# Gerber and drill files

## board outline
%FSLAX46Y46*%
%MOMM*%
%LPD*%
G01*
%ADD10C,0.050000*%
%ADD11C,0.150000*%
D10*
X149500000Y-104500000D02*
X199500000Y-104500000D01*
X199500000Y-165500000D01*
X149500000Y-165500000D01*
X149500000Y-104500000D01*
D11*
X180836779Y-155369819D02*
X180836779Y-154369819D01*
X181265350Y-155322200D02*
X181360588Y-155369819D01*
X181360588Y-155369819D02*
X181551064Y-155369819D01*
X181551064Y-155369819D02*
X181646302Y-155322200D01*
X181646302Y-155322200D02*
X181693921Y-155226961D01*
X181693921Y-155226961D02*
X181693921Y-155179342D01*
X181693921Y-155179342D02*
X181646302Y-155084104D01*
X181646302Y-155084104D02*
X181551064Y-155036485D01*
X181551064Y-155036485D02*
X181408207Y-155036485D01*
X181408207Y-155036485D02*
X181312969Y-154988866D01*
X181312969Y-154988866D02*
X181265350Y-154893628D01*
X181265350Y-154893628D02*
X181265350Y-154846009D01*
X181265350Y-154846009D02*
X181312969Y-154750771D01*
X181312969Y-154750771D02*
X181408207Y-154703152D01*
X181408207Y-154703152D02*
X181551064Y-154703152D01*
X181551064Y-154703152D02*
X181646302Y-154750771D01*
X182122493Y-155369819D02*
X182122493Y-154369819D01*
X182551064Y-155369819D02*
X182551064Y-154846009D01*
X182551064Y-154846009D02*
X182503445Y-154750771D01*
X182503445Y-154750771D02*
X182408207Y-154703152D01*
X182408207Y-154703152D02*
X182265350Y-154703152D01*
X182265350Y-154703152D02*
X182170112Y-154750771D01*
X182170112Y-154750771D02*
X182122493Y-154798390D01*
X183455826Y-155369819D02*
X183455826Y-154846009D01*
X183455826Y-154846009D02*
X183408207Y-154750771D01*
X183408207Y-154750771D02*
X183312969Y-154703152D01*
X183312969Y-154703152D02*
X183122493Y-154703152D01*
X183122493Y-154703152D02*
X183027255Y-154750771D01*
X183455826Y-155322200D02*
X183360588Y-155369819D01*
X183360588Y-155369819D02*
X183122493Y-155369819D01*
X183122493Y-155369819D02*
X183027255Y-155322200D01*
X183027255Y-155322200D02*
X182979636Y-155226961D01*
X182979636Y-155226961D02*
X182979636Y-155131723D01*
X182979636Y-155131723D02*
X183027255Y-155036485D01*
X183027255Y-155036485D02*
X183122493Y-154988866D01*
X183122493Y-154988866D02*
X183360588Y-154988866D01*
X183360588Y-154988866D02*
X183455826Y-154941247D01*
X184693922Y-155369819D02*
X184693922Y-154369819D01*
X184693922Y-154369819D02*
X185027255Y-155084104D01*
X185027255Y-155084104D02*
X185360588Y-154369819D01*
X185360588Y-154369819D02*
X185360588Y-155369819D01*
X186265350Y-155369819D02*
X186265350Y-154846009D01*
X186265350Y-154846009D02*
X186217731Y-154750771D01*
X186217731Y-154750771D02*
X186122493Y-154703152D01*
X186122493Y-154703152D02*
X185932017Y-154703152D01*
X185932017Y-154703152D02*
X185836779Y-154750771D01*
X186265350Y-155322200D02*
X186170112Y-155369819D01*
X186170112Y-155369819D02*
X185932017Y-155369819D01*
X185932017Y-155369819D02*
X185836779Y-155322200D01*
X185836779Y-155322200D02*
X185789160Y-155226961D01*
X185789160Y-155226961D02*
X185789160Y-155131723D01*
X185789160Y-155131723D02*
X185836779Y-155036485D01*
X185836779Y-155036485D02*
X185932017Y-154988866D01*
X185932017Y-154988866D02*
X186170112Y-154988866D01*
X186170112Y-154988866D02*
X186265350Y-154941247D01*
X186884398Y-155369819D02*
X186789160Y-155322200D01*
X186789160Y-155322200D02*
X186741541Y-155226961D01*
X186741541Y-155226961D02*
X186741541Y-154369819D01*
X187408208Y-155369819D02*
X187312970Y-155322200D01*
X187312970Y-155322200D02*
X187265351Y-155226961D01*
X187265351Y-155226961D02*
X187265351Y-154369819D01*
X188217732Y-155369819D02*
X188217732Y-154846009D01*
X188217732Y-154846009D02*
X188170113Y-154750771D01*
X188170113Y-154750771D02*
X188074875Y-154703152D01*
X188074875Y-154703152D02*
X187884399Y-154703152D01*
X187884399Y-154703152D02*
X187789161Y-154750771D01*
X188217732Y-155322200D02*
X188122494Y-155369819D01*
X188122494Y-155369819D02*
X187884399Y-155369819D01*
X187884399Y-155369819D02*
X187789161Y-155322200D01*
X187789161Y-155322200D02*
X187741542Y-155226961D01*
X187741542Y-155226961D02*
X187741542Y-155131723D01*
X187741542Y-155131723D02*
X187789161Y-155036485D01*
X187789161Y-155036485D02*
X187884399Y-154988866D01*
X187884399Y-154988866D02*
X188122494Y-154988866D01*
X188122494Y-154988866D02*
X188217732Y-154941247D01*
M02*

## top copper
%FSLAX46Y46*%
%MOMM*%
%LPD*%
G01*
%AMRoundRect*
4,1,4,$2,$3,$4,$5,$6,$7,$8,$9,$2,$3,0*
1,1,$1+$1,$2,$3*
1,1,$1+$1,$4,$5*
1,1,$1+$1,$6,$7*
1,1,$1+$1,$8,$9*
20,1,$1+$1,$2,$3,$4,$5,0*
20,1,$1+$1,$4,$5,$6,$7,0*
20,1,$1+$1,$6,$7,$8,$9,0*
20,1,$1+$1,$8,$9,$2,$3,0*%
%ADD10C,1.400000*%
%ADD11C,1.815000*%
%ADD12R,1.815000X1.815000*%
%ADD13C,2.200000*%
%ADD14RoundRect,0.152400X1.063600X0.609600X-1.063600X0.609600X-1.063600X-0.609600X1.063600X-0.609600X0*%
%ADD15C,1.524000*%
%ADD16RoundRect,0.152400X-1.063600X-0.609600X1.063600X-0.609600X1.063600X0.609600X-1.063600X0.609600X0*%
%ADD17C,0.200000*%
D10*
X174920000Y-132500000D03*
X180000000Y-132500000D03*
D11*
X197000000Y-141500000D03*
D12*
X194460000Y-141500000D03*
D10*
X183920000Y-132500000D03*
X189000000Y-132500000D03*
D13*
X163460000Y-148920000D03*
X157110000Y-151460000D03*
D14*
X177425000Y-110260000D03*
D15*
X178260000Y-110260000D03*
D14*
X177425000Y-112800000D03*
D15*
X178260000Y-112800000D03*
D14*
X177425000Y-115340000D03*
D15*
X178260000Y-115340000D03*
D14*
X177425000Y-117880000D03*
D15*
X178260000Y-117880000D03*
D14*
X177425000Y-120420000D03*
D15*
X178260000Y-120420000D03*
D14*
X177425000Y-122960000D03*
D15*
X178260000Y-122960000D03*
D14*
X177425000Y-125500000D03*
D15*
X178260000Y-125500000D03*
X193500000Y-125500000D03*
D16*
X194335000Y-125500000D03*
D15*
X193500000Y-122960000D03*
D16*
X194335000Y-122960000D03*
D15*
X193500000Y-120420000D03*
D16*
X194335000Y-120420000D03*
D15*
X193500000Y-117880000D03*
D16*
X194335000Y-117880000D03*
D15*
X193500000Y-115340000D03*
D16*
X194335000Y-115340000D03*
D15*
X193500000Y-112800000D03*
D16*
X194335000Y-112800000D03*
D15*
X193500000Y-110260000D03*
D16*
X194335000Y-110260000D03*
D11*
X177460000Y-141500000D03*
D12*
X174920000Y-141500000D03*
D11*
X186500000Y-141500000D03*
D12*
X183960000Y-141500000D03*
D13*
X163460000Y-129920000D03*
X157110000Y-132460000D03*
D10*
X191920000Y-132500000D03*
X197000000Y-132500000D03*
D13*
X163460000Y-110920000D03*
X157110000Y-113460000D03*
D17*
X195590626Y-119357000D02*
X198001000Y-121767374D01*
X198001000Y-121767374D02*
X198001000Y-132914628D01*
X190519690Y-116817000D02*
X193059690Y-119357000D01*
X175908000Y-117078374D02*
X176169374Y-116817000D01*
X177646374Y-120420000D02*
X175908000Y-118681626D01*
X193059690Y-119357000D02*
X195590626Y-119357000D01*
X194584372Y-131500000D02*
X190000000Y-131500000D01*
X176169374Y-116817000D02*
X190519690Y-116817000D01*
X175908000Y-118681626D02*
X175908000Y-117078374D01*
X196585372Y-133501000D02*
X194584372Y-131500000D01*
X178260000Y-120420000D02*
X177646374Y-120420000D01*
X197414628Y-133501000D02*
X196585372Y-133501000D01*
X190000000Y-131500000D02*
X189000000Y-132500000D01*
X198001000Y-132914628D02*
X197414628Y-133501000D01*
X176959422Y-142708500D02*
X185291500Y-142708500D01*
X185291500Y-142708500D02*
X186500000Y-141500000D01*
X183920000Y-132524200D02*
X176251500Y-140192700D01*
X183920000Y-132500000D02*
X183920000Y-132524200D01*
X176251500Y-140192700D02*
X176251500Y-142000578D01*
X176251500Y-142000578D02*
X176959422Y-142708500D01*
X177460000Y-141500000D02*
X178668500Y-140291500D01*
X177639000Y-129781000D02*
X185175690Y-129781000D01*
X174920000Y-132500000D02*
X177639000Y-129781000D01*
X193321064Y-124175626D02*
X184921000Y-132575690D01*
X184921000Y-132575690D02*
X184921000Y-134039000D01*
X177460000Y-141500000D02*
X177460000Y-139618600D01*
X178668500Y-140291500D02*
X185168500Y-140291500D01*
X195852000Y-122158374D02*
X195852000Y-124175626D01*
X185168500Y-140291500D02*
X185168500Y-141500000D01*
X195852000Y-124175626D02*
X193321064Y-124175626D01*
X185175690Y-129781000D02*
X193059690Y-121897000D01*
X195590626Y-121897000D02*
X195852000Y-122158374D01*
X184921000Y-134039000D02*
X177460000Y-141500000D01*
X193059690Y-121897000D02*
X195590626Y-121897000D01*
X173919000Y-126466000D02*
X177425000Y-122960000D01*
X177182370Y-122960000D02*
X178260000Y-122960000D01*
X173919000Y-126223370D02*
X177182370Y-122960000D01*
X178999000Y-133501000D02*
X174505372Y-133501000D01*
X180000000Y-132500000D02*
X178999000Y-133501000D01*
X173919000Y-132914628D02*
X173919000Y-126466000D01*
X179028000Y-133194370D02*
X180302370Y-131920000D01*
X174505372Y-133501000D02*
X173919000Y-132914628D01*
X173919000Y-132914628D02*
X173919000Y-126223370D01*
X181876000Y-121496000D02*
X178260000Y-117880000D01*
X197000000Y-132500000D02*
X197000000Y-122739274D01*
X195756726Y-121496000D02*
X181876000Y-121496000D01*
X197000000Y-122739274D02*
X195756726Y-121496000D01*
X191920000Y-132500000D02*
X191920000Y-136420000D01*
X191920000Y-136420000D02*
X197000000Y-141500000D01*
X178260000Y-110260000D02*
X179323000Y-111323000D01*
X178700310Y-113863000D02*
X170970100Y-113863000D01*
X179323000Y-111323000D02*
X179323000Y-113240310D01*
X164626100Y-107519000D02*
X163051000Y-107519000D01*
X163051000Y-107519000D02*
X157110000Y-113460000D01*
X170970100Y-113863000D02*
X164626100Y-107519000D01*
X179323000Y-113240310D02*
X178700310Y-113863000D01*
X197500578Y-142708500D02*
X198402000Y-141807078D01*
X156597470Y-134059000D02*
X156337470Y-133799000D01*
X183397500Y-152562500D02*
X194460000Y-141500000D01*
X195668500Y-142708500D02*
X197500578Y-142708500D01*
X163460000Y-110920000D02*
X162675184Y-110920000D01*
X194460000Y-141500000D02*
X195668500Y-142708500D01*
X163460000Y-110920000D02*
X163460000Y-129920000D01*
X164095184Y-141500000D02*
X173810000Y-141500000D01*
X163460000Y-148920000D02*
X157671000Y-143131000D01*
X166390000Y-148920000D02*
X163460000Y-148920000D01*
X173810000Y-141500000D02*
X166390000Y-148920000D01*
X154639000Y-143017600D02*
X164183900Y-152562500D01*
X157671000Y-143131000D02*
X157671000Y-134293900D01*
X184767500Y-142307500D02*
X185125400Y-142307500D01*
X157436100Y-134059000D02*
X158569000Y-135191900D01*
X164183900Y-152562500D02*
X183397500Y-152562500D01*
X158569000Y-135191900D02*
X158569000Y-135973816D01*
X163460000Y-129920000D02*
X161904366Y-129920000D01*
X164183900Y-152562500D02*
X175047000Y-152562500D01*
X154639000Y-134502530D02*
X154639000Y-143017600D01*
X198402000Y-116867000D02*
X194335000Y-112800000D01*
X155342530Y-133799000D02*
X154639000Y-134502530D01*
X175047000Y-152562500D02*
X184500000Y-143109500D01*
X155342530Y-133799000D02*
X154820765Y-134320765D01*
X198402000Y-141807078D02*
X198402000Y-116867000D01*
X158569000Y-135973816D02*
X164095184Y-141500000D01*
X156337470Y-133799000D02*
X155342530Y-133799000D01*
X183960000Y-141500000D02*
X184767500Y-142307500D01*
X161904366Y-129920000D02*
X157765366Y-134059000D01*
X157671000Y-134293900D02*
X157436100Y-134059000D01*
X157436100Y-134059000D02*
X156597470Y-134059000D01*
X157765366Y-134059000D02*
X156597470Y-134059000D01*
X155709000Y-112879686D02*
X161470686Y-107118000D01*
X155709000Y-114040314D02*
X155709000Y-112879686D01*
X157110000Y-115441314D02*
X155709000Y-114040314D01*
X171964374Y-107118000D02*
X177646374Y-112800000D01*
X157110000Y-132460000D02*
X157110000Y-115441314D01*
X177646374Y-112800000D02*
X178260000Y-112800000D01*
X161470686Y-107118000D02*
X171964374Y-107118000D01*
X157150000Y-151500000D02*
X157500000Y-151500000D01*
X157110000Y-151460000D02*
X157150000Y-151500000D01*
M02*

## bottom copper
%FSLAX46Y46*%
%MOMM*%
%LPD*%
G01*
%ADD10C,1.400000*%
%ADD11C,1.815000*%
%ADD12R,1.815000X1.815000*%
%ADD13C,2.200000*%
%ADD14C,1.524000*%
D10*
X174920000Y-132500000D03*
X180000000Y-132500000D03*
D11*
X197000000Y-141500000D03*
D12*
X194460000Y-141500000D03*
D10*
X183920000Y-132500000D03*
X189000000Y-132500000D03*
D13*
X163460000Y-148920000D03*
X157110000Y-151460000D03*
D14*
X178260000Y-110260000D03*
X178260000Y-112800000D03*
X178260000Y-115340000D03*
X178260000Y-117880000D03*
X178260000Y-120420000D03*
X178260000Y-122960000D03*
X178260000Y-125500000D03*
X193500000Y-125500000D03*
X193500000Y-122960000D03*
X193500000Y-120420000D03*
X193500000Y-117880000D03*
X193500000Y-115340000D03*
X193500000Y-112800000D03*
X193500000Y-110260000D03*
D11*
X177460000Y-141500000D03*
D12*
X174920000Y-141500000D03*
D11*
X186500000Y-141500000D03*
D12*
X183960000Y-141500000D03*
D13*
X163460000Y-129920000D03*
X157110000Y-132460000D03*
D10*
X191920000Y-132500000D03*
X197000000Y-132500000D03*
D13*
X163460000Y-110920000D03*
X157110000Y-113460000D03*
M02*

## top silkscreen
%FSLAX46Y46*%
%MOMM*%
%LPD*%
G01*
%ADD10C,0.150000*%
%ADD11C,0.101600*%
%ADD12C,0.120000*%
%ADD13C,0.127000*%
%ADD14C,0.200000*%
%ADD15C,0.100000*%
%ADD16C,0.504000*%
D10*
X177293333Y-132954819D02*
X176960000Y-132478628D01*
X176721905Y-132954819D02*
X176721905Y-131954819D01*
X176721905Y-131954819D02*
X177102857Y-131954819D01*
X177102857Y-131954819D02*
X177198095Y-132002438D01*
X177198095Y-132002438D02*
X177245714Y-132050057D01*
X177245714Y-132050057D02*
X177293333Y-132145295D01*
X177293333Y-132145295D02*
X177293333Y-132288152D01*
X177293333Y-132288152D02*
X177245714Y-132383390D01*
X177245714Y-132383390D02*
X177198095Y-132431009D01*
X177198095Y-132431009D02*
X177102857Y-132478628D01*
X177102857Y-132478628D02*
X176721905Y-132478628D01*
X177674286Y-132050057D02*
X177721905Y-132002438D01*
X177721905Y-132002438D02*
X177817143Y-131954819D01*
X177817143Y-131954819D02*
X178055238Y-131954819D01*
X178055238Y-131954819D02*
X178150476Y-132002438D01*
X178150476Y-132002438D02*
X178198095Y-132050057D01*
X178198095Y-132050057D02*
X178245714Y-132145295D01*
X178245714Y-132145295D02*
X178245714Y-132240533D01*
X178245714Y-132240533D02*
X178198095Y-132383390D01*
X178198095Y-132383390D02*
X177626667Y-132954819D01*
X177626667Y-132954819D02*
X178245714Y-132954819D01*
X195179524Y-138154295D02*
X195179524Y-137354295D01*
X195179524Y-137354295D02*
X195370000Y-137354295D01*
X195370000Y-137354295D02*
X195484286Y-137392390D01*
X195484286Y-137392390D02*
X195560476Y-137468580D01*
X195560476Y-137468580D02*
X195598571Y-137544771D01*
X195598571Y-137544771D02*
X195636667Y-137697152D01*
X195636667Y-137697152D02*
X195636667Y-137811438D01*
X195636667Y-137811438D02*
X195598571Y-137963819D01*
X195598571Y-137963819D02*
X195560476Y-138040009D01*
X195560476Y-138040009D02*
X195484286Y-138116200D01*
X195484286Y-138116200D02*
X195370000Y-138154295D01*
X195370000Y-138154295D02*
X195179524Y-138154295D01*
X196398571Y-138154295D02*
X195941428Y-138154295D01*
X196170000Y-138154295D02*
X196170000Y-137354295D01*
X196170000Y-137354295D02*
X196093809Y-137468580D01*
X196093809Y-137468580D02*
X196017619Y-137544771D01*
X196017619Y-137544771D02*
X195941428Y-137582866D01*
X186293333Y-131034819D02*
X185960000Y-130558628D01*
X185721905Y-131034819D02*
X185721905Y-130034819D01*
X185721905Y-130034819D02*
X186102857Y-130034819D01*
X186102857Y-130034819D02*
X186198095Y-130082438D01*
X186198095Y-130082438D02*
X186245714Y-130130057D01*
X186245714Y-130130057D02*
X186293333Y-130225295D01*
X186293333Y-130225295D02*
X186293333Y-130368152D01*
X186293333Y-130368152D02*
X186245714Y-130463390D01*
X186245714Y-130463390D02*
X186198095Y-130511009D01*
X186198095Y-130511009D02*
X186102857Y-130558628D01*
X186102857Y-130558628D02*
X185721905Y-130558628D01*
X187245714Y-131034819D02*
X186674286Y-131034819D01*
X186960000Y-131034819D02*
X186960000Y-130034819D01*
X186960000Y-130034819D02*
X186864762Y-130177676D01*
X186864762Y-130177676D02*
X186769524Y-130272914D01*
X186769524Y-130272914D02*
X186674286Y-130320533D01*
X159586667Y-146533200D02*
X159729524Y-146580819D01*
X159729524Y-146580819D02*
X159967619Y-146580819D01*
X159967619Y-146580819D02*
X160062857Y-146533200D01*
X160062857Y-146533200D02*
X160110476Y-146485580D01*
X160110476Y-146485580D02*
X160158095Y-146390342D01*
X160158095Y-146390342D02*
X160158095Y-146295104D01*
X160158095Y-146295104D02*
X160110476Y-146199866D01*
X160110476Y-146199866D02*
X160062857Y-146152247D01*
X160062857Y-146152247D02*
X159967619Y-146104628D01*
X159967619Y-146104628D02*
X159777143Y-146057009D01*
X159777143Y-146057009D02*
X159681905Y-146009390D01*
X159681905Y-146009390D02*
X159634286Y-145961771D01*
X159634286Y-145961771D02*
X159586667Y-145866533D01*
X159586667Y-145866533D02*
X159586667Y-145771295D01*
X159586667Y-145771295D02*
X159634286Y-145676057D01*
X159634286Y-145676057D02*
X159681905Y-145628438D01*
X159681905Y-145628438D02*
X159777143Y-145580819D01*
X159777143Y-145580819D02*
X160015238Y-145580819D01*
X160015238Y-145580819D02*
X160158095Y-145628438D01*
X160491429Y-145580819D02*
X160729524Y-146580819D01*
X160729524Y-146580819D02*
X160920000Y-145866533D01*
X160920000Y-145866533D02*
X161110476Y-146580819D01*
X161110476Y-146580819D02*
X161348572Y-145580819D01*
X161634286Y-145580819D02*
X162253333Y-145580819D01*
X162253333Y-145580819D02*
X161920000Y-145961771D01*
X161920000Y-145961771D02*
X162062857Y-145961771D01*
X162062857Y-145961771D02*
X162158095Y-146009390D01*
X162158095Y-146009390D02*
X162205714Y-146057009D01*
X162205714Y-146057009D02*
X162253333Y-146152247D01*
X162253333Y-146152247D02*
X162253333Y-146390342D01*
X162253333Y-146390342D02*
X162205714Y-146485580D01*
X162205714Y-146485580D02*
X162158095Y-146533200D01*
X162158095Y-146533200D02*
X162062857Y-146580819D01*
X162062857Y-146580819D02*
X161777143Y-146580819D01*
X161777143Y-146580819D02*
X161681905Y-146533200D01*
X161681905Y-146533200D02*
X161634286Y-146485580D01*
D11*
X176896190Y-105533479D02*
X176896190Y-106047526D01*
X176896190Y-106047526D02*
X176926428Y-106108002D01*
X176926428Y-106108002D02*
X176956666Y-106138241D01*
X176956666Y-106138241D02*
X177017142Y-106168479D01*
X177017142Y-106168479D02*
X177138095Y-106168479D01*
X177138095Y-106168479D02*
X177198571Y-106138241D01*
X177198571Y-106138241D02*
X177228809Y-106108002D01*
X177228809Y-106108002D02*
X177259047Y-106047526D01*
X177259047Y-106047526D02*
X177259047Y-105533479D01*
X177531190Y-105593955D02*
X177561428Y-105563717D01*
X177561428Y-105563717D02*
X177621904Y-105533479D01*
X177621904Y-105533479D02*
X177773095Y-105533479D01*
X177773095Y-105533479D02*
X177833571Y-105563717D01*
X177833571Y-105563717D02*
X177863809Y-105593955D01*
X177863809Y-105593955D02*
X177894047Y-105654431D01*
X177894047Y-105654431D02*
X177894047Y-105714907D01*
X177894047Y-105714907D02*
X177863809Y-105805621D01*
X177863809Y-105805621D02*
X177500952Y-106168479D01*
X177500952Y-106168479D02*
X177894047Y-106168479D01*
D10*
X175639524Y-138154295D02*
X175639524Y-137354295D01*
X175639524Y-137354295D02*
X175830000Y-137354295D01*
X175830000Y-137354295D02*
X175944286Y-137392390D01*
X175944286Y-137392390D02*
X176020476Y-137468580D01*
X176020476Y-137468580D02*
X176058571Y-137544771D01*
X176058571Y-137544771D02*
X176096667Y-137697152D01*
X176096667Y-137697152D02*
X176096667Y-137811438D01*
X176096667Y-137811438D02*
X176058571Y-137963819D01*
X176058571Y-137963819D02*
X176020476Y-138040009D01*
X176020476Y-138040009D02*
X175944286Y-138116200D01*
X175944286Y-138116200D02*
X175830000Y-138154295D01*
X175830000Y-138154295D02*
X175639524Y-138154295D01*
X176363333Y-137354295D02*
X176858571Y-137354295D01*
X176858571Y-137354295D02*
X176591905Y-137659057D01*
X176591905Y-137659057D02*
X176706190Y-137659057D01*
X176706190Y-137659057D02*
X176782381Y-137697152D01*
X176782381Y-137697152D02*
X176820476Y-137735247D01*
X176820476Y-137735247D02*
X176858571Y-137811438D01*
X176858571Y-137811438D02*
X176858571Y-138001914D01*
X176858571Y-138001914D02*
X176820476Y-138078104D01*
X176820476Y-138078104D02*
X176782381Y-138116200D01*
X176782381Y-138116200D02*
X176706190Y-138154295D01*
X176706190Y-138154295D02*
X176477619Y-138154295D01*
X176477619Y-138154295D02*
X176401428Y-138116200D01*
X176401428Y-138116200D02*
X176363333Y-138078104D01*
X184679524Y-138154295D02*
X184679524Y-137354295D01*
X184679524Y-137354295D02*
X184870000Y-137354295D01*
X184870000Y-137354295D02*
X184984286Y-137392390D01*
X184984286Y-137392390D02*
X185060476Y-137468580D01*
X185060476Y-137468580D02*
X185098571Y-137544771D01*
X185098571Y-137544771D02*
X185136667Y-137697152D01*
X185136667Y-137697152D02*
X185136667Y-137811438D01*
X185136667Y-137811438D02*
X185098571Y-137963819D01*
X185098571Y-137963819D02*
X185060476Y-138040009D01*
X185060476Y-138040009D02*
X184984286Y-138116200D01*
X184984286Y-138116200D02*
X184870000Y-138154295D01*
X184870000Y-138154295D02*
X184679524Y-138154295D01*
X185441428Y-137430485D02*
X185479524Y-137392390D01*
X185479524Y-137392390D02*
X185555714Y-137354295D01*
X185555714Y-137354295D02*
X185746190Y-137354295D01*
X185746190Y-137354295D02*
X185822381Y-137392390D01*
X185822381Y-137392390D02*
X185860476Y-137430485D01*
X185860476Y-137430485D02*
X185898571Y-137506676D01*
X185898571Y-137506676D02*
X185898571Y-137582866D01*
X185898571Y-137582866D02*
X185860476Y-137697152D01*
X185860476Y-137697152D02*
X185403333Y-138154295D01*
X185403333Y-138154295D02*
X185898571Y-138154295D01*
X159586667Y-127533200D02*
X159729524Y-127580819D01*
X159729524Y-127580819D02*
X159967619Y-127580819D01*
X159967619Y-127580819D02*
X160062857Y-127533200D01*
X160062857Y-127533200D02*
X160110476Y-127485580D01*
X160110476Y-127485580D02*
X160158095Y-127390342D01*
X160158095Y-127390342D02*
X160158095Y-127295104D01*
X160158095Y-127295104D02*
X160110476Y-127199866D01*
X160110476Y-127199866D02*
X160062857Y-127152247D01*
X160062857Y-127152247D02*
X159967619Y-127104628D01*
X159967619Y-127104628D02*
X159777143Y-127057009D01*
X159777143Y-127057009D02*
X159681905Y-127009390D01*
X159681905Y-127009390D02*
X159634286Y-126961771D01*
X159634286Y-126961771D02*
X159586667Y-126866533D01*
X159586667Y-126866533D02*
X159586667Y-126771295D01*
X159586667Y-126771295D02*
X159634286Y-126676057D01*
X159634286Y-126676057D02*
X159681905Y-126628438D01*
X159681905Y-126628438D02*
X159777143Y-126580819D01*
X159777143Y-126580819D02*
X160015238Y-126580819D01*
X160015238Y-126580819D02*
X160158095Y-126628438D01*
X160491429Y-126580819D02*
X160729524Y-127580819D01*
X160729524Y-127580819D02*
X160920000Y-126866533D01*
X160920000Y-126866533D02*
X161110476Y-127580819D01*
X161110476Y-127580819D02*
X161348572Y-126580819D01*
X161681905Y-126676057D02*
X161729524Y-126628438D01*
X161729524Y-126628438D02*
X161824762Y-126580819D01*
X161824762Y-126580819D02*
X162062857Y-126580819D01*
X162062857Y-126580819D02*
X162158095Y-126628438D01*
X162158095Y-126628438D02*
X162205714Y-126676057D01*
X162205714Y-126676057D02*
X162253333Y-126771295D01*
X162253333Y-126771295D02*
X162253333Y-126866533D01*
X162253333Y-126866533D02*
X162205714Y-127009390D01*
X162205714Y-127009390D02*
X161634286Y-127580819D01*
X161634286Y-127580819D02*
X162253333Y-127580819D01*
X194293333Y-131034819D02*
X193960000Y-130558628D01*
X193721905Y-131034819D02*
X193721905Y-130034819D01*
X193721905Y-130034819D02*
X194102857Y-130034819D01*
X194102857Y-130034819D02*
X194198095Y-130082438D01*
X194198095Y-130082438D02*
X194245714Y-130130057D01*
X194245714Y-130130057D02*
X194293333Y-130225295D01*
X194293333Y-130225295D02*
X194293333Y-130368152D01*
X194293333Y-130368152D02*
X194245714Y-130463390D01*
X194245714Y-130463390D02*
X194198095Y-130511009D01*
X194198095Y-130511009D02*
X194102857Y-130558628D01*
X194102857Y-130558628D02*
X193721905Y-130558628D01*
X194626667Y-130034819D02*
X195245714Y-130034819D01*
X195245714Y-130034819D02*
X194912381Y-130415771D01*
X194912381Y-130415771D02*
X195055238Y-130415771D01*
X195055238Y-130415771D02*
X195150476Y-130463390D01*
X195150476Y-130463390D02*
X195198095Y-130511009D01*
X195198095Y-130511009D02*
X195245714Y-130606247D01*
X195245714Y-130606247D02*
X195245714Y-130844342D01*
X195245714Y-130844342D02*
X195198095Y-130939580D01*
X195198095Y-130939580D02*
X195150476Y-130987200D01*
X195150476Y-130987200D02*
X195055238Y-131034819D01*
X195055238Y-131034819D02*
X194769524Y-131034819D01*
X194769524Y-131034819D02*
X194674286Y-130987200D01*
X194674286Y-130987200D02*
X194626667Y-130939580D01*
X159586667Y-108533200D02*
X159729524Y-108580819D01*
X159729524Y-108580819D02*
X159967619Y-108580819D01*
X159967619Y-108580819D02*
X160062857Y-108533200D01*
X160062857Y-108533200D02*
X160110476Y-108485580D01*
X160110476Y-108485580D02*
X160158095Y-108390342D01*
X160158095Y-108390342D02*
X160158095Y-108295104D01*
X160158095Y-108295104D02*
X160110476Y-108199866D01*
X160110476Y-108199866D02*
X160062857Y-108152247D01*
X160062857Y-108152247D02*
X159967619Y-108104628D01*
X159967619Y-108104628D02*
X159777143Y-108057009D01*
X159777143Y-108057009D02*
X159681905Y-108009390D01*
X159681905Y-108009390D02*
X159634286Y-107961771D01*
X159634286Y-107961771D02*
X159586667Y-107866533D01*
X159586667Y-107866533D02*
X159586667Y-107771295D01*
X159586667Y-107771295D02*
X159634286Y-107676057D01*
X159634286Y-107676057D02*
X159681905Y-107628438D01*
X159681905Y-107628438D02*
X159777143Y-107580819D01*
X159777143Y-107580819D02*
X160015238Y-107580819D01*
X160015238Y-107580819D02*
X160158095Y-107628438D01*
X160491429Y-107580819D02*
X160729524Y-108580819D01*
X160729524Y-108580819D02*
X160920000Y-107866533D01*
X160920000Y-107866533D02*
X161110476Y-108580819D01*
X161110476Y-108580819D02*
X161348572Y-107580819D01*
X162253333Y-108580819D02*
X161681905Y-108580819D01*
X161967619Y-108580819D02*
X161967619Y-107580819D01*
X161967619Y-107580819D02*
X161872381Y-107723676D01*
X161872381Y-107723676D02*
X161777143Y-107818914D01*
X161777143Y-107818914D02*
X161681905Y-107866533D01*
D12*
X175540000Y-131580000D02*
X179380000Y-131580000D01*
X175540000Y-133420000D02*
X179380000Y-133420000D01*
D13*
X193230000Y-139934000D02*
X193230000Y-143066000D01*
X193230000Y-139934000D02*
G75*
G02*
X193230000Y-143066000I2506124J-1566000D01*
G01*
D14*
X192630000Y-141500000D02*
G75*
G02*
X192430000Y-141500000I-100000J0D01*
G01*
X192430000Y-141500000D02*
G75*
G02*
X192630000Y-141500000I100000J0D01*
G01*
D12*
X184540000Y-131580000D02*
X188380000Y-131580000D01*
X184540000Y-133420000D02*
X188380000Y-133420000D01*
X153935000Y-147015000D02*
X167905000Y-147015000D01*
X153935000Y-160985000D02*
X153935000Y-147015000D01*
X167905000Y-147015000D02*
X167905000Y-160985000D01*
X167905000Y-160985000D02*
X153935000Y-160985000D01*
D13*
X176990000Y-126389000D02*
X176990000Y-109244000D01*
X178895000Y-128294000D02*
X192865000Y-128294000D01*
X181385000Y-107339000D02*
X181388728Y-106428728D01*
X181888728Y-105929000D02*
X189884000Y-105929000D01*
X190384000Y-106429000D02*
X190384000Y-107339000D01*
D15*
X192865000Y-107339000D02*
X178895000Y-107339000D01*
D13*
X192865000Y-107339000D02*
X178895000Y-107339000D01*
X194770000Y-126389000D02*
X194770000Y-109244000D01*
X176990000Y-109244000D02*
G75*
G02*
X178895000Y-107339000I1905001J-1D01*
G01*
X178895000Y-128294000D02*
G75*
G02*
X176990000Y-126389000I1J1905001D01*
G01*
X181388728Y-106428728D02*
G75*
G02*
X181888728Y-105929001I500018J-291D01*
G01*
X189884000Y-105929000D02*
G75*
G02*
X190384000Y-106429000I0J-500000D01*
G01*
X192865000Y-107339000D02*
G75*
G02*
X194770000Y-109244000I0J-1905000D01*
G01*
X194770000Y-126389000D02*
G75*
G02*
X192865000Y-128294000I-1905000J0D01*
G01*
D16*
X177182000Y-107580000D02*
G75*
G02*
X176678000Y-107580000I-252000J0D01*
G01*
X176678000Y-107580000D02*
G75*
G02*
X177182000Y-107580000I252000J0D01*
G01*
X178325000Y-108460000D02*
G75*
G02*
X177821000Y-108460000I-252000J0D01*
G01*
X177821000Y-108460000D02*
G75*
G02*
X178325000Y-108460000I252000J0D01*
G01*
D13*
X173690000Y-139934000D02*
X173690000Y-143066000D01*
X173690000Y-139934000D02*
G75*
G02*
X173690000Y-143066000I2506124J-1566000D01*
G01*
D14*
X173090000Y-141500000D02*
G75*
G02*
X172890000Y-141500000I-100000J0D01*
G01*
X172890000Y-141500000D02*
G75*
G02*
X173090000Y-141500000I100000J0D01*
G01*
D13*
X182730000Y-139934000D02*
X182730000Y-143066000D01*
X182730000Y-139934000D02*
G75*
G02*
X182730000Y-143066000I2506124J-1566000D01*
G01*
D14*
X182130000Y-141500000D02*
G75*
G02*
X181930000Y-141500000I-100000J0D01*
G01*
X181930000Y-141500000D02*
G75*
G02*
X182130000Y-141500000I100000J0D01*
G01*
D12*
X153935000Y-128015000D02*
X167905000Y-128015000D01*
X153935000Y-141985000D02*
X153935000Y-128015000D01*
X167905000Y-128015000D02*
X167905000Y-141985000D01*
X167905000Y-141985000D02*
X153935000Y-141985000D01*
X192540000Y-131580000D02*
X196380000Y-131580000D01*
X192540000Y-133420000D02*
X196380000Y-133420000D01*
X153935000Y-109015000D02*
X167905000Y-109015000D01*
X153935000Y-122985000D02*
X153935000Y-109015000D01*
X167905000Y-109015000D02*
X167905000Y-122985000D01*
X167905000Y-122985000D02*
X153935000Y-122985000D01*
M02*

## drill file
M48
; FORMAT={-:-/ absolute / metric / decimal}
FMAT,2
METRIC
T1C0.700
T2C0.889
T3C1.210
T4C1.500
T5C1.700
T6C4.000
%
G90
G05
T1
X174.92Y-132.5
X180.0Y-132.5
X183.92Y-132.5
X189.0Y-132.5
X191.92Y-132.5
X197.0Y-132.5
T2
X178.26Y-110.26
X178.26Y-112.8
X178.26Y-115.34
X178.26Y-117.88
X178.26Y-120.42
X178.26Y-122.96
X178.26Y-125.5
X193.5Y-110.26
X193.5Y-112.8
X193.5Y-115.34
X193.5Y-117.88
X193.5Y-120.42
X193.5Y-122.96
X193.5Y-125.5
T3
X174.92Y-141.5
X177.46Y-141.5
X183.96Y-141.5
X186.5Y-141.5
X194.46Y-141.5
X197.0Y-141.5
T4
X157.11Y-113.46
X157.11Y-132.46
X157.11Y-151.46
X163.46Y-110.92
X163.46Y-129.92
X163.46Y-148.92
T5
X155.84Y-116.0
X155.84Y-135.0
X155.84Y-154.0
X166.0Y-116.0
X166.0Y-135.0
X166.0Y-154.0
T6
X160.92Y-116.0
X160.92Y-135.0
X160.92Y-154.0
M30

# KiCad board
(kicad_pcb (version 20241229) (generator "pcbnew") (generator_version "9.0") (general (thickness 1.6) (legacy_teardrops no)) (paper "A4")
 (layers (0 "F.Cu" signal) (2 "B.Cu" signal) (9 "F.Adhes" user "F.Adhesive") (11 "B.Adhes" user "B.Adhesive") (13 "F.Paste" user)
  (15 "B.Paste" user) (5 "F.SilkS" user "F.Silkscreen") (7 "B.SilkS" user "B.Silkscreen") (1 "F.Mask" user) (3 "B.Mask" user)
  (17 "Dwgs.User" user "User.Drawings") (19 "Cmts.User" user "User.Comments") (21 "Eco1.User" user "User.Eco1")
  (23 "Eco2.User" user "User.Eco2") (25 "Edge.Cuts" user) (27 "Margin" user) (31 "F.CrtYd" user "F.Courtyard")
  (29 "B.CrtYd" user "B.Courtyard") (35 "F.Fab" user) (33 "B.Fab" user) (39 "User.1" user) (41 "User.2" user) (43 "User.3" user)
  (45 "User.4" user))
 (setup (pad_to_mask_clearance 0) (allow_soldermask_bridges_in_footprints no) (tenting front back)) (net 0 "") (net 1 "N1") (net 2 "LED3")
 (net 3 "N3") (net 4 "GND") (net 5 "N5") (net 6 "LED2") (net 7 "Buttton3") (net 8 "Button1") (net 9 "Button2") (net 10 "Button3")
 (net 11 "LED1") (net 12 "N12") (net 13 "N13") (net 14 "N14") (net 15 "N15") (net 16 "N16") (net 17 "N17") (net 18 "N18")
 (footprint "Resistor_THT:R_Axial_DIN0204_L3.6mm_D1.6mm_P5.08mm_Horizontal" (layer "F.Cu") (at 174.92 132.5)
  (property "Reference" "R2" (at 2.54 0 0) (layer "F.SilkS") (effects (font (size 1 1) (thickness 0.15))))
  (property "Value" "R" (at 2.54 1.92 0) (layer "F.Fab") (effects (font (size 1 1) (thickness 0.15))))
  (fp_line (start 0.62 -0.92) (end 4.46 -0.92) (stroke (width 0.12) (type solid)) (layer "F.SilkS"))
  (fp_line (start 0.62 0.92) (end 4.46 0.92) (stroke (width 0.12) (type solid)) (layer "F.SilkS"))
  (pad "1" thru_hole circle (at 0 0) (size 1.4 1.4) (drill 0.7) (layers "*.Cu" "*.Mask") (remove_unused_layers no) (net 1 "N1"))
  (pad "2" thru_hole circle (at 5.08 0) (size 1.4 1.4) (drill 0.7) (layers "*.Cu" "*.Mask") (remove_unused_layers no) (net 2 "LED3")))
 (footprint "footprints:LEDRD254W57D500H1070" (layer "F.Cu") (at 195.73 141.5)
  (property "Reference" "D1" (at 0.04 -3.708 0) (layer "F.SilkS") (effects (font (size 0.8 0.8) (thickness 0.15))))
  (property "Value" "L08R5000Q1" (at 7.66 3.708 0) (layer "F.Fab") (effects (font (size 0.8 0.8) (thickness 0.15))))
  (fp_line (start -2.5 -1.566) (end -2.5 1.566) (stroke (width 0.127) (type solid)) (layer "F.SilkS"))
  (fp_arc (start -2.5 -1.566) (mid 2.961291 0) (end -2.5 1.566) (stroke (width 0.127) (type solid)) (layer "F.SilkS"))
  (fp_circle (center -3.2 0) (end -3.1 0) (stroke (width 0.2) (type solid)) (fill no) (layer "F.SilkS"))
  (pad "A" thru_hole circle (at 1.27 0) (size 1.815 1.815) (drill 1.21) (layers "*.Cu" "*.Mask") (remove_unused_layers no) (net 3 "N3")
   (solder_mask_margin 0.102))
  (pad "C" thru_hole rect (at -1.27 0) (size 1.815 1.815) (drill 1.21) (layers "*.Cu" "*.Mask") (remove_unused_layers no) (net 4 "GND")
   (solder_mask_margin 0.102)))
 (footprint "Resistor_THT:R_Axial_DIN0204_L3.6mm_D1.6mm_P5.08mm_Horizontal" (layer "F.Cu") (at 183.92 132.5)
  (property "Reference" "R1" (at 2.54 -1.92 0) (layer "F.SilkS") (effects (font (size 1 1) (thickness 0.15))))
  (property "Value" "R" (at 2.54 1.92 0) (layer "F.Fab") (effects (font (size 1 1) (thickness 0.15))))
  (fp_line (start 0.62 -0.92) (end 4.46 -0.92) (stroke (width 0.12) (type solid)) (layer "F.SilkS"))
  (fp_line (start 0.62 0.92) (end 4.46 0.92) (stroke (width 0.12) (type solid)) (layer "F.SilkS"))
  (pad "1" thru_hole circle (at 0 0) (size 1.4 1.4) (drill 0.7) (layers "*.Cu" "*.Mask") (remove_unused_layers no) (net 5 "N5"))
  (pad "2" thru_hole circle (at 5.08 0) (size 1.4 1.4) (drill 0.7) (layers "*.Cu" "*.Mask") (remove_unused_layers no) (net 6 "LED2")))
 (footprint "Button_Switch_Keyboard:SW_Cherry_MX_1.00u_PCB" (layer "F.Cu") (at 163.46 148.92)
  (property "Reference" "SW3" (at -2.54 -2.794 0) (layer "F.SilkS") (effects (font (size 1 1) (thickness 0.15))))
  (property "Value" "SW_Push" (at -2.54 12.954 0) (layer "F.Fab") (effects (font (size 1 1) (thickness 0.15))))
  (fp_line (start -9.525 -1.905) (end 4.445 -1.905) (stroke (width 0.12) (type solid)) (layer "F.SilkS"))
  (fp_line (start -9.525 12.065) (end -9.525 -1.905) (stroke (width 0.12) (type solid)) (layer "F.SilkS"))
  (fp_line (start 4.445 -1.905) (end 4.445 12.065) (stroke (width 0.12) (type solid)) (layer "F.SilkS"))
  (fp_line (start 4.445 12.065) (end -9.525 12.065) (stroke (width 0.12) (type solid)) (layer "F.SilkS"))
  (pad "" np_thru_hole circle (at -7.62 5.08) (size 1.7 1.7) (drill 1.7) (layers "*.Cu" "*.Mask"))
  (pad "" np_thru_hole circle (at -2.54 5.08) (size 4 4) (drill 4) (layers "*.Cu" "*.Mask"))
  (pad "" np_thru_hole circle (at 2.54 5.08) (size 1.7 1.7) (drill 1.7) (layers "*.Cu" "*.Mask"))
  (pad "1" thru_hole circle (at 0 0) (size 2.2 2.2) (drill 1.5) (layers "*.Cu" "*.Mask") (remove_unused_layers no) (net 4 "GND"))
  (pad "2" thru_hole circle (at -6.35 2.54) (size 2.2 2.2) (drill 1.5) (layers "*.Cu" "*.Mask") (remove_unused_layers no) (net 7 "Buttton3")))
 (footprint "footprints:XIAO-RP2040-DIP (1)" (layer "F.Cu") (at 185.88 117.88)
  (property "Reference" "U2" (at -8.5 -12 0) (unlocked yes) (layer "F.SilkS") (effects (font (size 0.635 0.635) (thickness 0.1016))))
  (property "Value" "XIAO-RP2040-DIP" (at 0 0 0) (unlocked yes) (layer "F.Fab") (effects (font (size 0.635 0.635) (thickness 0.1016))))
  (fp_line (start -8.89 8.509) (end -8.89 -8.636) (stroke (width 0.127) (type solid)) (layer "F.SilkS"))
  (fp_line (start -6.985 10.414) (end 6.985 10.414) (stroke (width 0.127) (type solid)) (layer "F.SilkS"))
  (fp_line (start -4.495 -10.541) (end -4.491272 -11.451272) (stroke (width 0.127) (type solid)) (layer "F.SilkS"))
  (fp_line (start -3.991272 -11.951) (end 4.004 -11.951) (stroke (width 0.127) (type solid)) (layer "F.SilkS"))
  (fp_line (start 4.504 -11.451) (end 4.504 -10.541) (stroke (width 0.127) (type solid)) (layer "F.SilkS"))
  (fp_line (start 6.985 -10.541) (end -6.985 -10.541) (stroke (width 0.1) (type solid)) (layer "F.SilkS"))
  (fp_line (start 6.985 -10.541) (end -6.985 -10.541) (stroke (width 0.127) (type solid)) (layer "F.SilkS"))
  (fp_line (start 8.89 8.509) (end 8.89 -8.636) (stroke (width 0.127) (type solid)) (layer "F.SilkS"))
  (fp_arc (start -8.89 -8.636) (mid -8.332038 -9.983038) (end -6.985 -10.541) (stroke (width 0.127) (type solid)) (layer "F.SilkS"))
  (fp_arc (start -6.985 10.414) (mid -8.332038 9.856038) (end -8.89 8.509) (stroke (width 0.127) (type solid)) (layer "F.SilkS"))
  (fp_arc (start -4.491272 -11.451272) (mid -4.344728 -11.80464) (end -3.991272 -11.951) (stroke (width 0.127) (type default))
   (layer "F.SilkS"))
  (fp_arc (start 4.004 -11.951) (mid 4.357553 -11.804553) (end 4.504 -11.451) (stroke (width 0.127) (type default)) (layer "F.SilkS"))
  (fp_arc (start 6.985 -10.541) (mid 8.332038 -9.983038) (end 8.89 -8.636) (stroke (width 0.127) (type solid)) (layer "F.SilkS"))
  (fp_arc (start 8.89 8.509) (mid 8.332038 9.856038) (end 6.985 10.414) (stroke (width 0.127) (type solid)) (layer "F.SilkS"))
  (fp_circle (center -8.95 -10.3) (end -8.95 -10.554) (stroke (width 0.5) (type solid)) (fill yes) (layer "F.SilkS"))
  (fp_circle (center -7.807 -9.42) (end -7.807 -9.674) (stroke (width 0.5) (type solid)) (fill yes) (layer "F.SilkS"))
  (pad "1" smd roundrect (at -8.455 -7.62 180) (size 2.432 1.524) (layers "F.Cu" "F.Mask") (roundrect_rratio 0.1) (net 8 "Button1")
   (thermal_bridge_angle 45))
  (pad "1" thru_hole circle (at -7.62 -7.62 180) (size 1.524 1.524) (drill 0.889) (layers "*.Cu" "*.Mask") (remove_unused_layers no)
   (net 8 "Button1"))
  (pad "2" smd roundrect (at -8.455 -5.08 180) (size 2.432 1.524) (layers "F.Cu" "F.Mask") (roundrect_rratio 0.1) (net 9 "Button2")
   (thermal_bridge_angle 45))
  (pad "2" thru_hole circle (at -7.62 -5.08 180) (size 1.524 1.524) (drill 0.889) (layers "*.Cu" "*.Mask") (remove_unused_layers no)
   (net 9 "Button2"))
  (pad "3" smd roundrect (at -8.455 -2.54 180) (size 2.432 1.524) (layers "F.Cu" "F.Mask") (roundrect_rratio 0.1) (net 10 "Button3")
   (thermal_bridge_angle 45))
  (pad "3" thru_hole circle (at -7.62 -2.54 180) (size 1.524 1.524) (drill 0.889) (layers "*.Cu" "*.Mask") (remove_unused_layers no)
   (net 10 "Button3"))
  (pad "4" smd roundrect (at -8.455 0 180) (size 2.432 1.524) (layers "F.Cu" "F.Mask") (roundrect_rratio 0.1) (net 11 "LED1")
   (thermal_bridge_angle 45))
  (pad "4" thru_hole circle (at -7.62 0 180) (size 1.524 1.524) (drill 0.889) (layers "*.Cu" "*.Mask") (remove_unused_layers no)
   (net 11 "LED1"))
  (pad "5" smd roundrect (at -8.455 2.54 180) (size 2.432 1.524) (layers "F.Cu" "F.Mask") (roundrect_rratio 0.1) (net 6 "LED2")
   (thermal_bridge_angle 45))
  (pad "5" thru_hole circle (at -7.62 2.54 180) (size 1.524 1.524) (drill 0.889) (layers "*.Cu" "*.Mask") (remove_unused_layers no)
   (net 6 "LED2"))
  (pad "6" smd roundrect (at -8.455 5.08 180) (size 2.432 1.524) (layers "F.Cu" "F.Mask") (roundrect_rratio 0.1) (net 2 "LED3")
   (thermal_bridge_angle 45))
  (pad "6" thru_hole circle (at -7.62 5.08 180) (size 1.524 1.524) (drill 0.889) (layers "*.Cu" "*.Mask") (remove_unused_layers no)
   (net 2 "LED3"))
  (pad "7" smd roundrect (at -8.455 7.62 180) (size 2.432 1.524) (layers "F.Cu" "F.Mask") (roundrect_rratio 0.1) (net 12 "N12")
   (thermal_bridge_angle 45))
  (pad "7" thru_hole circle (at -7.62 7.62 180) (size 1.524 1.524) (drill 0.889) (layers "*.Cu" "*.Mask") (remove_unused_layers no)
   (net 12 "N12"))
  (pad "8" thru_hole circle (at 7.62 7.62) (size 1.524 1.524) (drill 0.889) (layers "*.Cu" "*.Mask") (remove_unused_layers no)
   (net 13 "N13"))
  (pad "8" smd roundrect (at 8.455 7.62) (size 2.432 1.524) (layers "F.Cu" "F.Mask") (roundrect_rratio 0.1) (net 13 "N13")
   (thermal_bridge_angle 45))
  (pad "9" thru_hole circle (at 7.62 5.08) (size 1.524 1.524) (drill 0.889) (layers "*.Cu" "*.Mask") (remove_unused_layers no)
   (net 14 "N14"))
  (pad "9" smd roundrect (at 8.455 5.08) (size 2.432 1.524) (layers "F.Cu" "F.Mask") (roundrect_rratio 0.1) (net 14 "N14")
   (thermal_bridge_angle 45))
  (pad "10" thru_hole circle (at 7.62 2.54) (size 1.524 1.524) (drill 0.889) (layers "*.Cu" "*.Mask") (remove_unused_layers no)
   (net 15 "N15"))
  (pad "10" smd roundrect (at 8.455 2.54) (size 2.432 1.524) (layers "F.Cu" "F.Mask") (roundrect_rratio 0.1) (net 15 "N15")
   (thermal_bridge_angle 45))
  (pad "11" thru_hole circle (at 7.62 0) (size 1.524 1.524) (drill 0.889) (layers "*.Cu" "*.Mask") (remove_unused_layers no) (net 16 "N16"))
  (pad "11" smd roundrect (at 8.455 0) (size 2.432 1.524) (layers "F.Cu" "F.Mask") (roundrect_rratio 0.1) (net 16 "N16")
   (thermal_bridge_angle 45))
  (pad "12" thru_hole circle (at 7.62 -2.54) (size 1.524 1.524) (drill 0.889) (layers "*.Cu" "*.Mask") (remove_unused_layers no)
   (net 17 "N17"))
  (pad "12" smd roundrect (at 8.455 -2.54) (size 2.432 1.524) (layers "F.Cu" "F.Mask") (roundrect_rratio 0.1) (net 17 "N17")
   (thermal_bridge_angle 45))
  (pad "13" thru_hole circle (at 7.62 -5.08) (size 1.524 1.524) (drill 0.889) (layers "*.Cu" "*.Mask") (remove_unused_layers no)
   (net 4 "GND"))
  (pad "13" smd roundrect (at 8.455 -5.08) (size 2.432 1.524) (layers "F.Cu" "F.Mask") (roundrect_rratio 0.1) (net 4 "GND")
   (thermal_bridge_angle 45))
  (pad "14" thru_hole circle (at 7.62 -7.62) (size 1.524 1.524) (drill 0.889) (layers "*.Cu" "*.Mask") (remove_unused_layers no)
   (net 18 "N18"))
  (pad "14" smd roundrect (at 8.455 -7.62) (size 2.432 1.524) (layers "F.Cu" "F.Mask") (roundrect_rratio 0.1) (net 18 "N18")
   (thermal_bridge_angle 45)))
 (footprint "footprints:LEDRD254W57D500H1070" (layer "F.Cu") (at 176.19 141.5)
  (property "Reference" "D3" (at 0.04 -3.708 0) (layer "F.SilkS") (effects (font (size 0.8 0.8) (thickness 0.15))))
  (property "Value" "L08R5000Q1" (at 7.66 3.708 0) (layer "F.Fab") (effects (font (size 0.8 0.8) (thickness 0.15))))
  (fp_line (start -2.5 -1.566) (end -2.5 1.566) (stroke (width 0.127) (type solid)) (layer "F.SilkS"))
  (fp_arc (start -2.5 -1.566) (mid 2.961291 0) (end -2.5 1.566) (stroke (width 0.127) (type solid)) (layer "F.SilkS"))
  (fp_circle (center -3.2 0) (end -3.1 0) (stroke (width 0.2) (type solid)) (fill no) (layer "F.SilkS"))
  (pad "A" thru_hole circle (at 1.27 0) (size 1.815 1.815) (drill 1.21) (layers "*.Cu" "*.Mask") (remove_unused_layers no) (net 1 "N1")
   (solder_mask_margin 0.102))
  (pad "C" thru_hole rect (at -1.27 0) (size 1.815 1.815) (drill 1.21) (layers "*.Cu" "*.Mask") (remove_unused_layers no) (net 4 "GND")
   (solder_mask_margin 0.102)))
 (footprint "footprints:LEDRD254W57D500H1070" (layer "F.Cu") (at 185.23 141.5)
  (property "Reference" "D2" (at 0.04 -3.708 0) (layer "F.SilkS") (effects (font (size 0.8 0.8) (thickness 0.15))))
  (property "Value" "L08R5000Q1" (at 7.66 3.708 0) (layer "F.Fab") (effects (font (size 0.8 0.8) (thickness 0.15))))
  (fp_line (start -2.5 -1.566) (end -2.5 1.566) (stroke (width 0.127) (type solid)) (layer "F.SilkS"))
  (fp_arc (start -2.5 -1.566) (mid 2.961291 0) (end -2.5 1.566) (stroke (width 0.127) (type solid)) (layer "F.SilkS"))
  (fp_circle (center -3.2 0) (end -3.1 0) (stroke (width 0.2) (type solid)) (fill no) (layer "F.SilkS"))
  (pad "A" thru_hole circle (at 1.27 0) (size 1.815 1.815) (drill 1.21) (layers "*.Cu" "*.Mask") (remove_unused_layers no) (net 5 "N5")
   (solder_mask_margin 0.102))
  (pad "C" thru_hole rect (at -1.27 0) (size 1.815 1.815) (drill 1.21) (layers "*.Cu" "*.Mask") (remove_unused_layers no) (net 4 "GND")
   (solder_mask_margin 0.102)))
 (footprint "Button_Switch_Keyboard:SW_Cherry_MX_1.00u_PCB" (layer "F.Cu") (at 163.46 129.92)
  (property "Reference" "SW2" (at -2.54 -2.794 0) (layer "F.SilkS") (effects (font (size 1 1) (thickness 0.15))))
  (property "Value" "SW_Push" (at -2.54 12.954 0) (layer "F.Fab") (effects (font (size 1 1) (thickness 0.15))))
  (fp_line (start -9.525 -1.905) (end 4.445 -1.905) (stroke (width 0.12) (type solid)) (layer "F.SilkS"))
  (fp_line (start -9.525 12.065) (end -9.525 -1.905) (stroke (width 0.12) (type solid)) (layer "F.SilkS"))
  (fp_line (start 4.445 -1.905) (end 4.445 12.065) (stroke (width 0.12) (type solid)) (layer "F.SilkS"))
  (fp_line (start 4.445 12.065) (end -9.525 12.065) (stroke (width 0.12) (type solid)) (layer "F.SilkS"))
  (pad "" np_thru_hole circle (at -7.62 5.08) (size 1.7 1.7) (drill 1.7) (layers "*.Cu" "*.Mask"))
  (pad "" np_thru_hole circle (at -2.54 5.08) (size 4 4) (drill 4) (layers "*.Cu" "*.Mask"))
  (pad "" np_thru_hole circle (at 2.54 5.08) (size 1.7 1.7) (drill 1.7) (layers "*.Cu" "*.Mask"))
  (pad "1" thru_hole circle (at 0 0) (size 2.2 2.2) (drill 1.5) (layers "*.Cu" "*.Mask") (remove_unused_layers no) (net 4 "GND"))
  (pad "2" thru_hole circle (at -6.35 2.54) (size 2.2 2.2) (drill 1.5) (layers "*.Cu" "*.Mask") (remove_unused_layers no) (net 9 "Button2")))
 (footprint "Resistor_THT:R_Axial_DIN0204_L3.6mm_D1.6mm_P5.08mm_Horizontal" (layer "F.Cu") (at 191.92 132.5)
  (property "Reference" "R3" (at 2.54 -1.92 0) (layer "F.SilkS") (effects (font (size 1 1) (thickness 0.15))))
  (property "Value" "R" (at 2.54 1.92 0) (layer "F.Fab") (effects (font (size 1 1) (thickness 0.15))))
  (fp_line (start 0.62 -0.92) (end 4.46 -0.92) (stroke (width 0.12) (type solid)) (layer "F.SilkS"))
  (fp_line (start 0.62 0.92) (end 4.46 0.92) (stroke (width 0.12) (type solid)) (layer "F.SilkS"))
  (pad "1" thru_hole circle (at 0 0) (size 1.4 1.4) (drill 0.7) (layers "*.Cu" "*.Mask") (remove_unused_layers no) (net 3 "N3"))
  (pad "2" thru_hole circle (at 5.08 0) (size 1.4 1.4) (drill 0.7) (layers "*.Cu" "*.Mask") (remove_unused_layers no) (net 11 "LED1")))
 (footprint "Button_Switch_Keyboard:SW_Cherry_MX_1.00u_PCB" (layer "F.Cu") (at 163.46 110.92)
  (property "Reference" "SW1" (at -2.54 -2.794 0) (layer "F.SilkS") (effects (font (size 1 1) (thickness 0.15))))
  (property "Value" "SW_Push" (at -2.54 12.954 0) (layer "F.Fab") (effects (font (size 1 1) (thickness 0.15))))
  (fp_line (start -9.525 -1.905) (end 4.445 -1.905) (stroke (width 0.12) (type solid)) (layer "F.SilkS"))
  (fp_line (start -9.525 12.065) (end -9.525 -1.905) (stroke (width 0.12) (type solid)) (layer "F.SilkS"))
  (fp_line (start 4.445 -1.905) (end 4.445 12.065) (stroke (width 0.12) (type solid)) (layer "F.SilkS"))
  (fp_line (start 4.445 12.065) (end -9.525 12.065) (stroke (width 0.12) (type solid)) (layer "F.SilkS"))
  (pad "" np_thru_hole circle (at -7.62 5.08) (size 1.7 1.7) (drill 1.7) (layers "*.Cu" "*.Mask"))
  (pad "" np_thru_hole circle (at -2.54 5.08) (size 4 4) (drill 4) (layers "*.Cu" "*.Mask"))
  (pad "" np_thru_hole circle (at 2.54 5.08) (size 1.7 1.7) (drill 1.7) (layers "*.Cu" "*.Mask"))
  (pad "1" thru_hole circle (at 0 0) (size 2.2 2.2) (drill 1.5) (layers "*.Cu" "*.Mask") (remove_unused_layers no) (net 4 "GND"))
  (pad "2" thru_hole circle (at -6.35 2.54) (size 2.2 2.2) (drill 1.5) (layers "*.Cu" "*.Mask") (remove_unused_layers no) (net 8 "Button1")))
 (gr_rect (start 149.5 104.5) (end 199.5 165.5) (stroke (width 0.05) (type default)) (fill no) (layer "Edge.Cuts"))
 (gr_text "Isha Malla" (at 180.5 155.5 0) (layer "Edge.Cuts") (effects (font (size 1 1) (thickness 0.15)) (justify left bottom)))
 (segment (start 195.590626 119.357) (end 198.001 121.767374) (width 0.2) (layer "F.Cu") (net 6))
 (segment (start 198.001 121.767374) (end 198.001 132.914628) (width 0.2) (layer "F.Cu") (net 6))
 (segment (start 190.51969 116.817) (end 193.05969 119.357) (width 0.2) (layer "F.Cu") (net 6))
 (segment (start 175.908 117.078374) (end 176.169374 116.817) (width 0.2) (layer "F.Cu") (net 6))
 (segment (start 177.646374 120.42) (end 175.908 118.681626) (width 0.2) (layer "F.Cu") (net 6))
 (segment (start 193.05969 119.357) (end 195.590626 119.357) (width 0.2) (layer "F.Cu") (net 6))
 (segment (start 194.584372 131.5) (end 190 131.5) (width 0.2) (layer "F.Cu") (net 6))
 (segment (start 176.169374 116.817) (end 190.51969 116.817) (width 0.2) (layer "F.Cu") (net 6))
 (segment (start 175.908 118.681626) (end 175.908 117.078374) (width 0.2) (layer "F.Cu") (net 6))
 (segment (start 196.585372 133.501) (end 194.584372 131.5) (width 0.2) (layer "F.Cu") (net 6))
 (segment (start 178.26 120.42) (end 177.646374 120.42) (width 0.2) (layer "F.Cu") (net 6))
 (segment (start 197.414628 133.501) (end 196.585372 133.501) (width 0.2) (layer "F.Cu") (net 6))
 (segment (start 190 131.5) (end 189 132.5) (width 0.2) (layer "F.Cu") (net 6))
 (segment (start 198.001 132.914628) (end 197.414628 133.501) (width 0.2) (layer "F.Cu") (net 6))
 (segment (start 176.959422 142.7085) (end 185.2915 142.7085) (width 0.2) (layer "F.Cu") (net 5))
 (segment (start 185.2915 142.7085) (end 186.5 141.5) (width 0.2) (layer "F.Cu") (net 5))
 (segment (start 183.92 132.5242) (end 176.2515 140.1927) (width 0.2) (layer "F.Cu") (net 5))
 (segment (start 183.92 132.5) (end 183.92 132.5242) (width 0.2) (layer "F.Cu") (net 5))
 (segment (start 176.2515 140.1927) (end 176.2515 142.000578) (width 0.2) (layer "F.Cu") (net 5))
 (segment (start 176.2515 142.000578) (end 176.959422 142.7085) (width 0.2) (layer "F.Cu") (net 5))
 (segment (start 177.46 141.5) (end 178.6685 140.2915) (width 0.2) (layer "F.Cu") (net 1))
 (segment (start 177.639 129.781) (end 185.17569 129.781) (width 0.2) (layer "F.Cu") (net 1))
 (segment (start 174.92 132.5) (end 177.639 129.781) (width 0.2) (layer "F.Cu") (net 1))
 (segment (start 193.321064 124.175626) (end 184.921 132.57569) (width 0.2) (layer "F.Cu") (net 1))
 (segment (start 184.921 132.57569) (end 184.921 134.039) (width 0.2) (layer "F.Cu") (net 1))
 (segment (start 177.46 141.5) (end 177.46 139.6186) (width 0.2) (layer "F.Cu") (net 1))
 (segment (start 178.6685 140.2915) (end 185.1685 140.2915) (width 0.2) (layer "F.Cu") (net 1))
 (segment (start 195.852 122.158374) (end 195.852 124.175626) (width 0.2) (layer "F.Cu") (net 1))
 (segment (start 185.1685 140.2915) (end 185.1685 141.5) (width 0.2) (layer "F.Cu") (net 1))
 (segment (start 195.852 124.175626) (end 193.321064 124.175626) (width 0.2) (layer "F.Cu") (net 1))
 (segment (start 185.17569 129.781) (end 193.05969 121.897) (width 0.2) (layer "F.Cu") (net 1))
 (segment (start 195.590626 121.897) (end 195.852 122.158374) (width 0.2) (layer "F.Cu") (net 1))
 (segment (start 184.921 134.039) (end 177.46 141.5) (width 0.2) (layer "F.Cu") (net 1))
 (segment (start 193.05969 121.897) (end 195.590626 121.897) (width 0.2) (layer "F.Cu") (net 1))
 (segment (start 173.919 126.466) (end 177.425 122.96) (width 0.2) (layer "F.Cu") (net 2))
 (segment (start 177.18237 122.96) (end 178.26 122.96) (width 0.2) (layer "F.Cu") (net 2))
 (segment (start 173.919 126.22337) (end 177.18237 122.96) (width 0.2) (layer "F.Cu") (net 2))
 (segment (start 178.999 133.501) (end 174.505372 133.501) (width 0.2) (layer "F.Cu") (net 2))
 (segment (start 180 132.5) (end 178.999 133.501) (width 0.2) (layer "F.Cu") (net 2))
 (segment (start 173.919 132.914628) (end 173.919 126.466) (width 0.2) (layer "F.Cu") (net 2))
 (segment (start 179.028 133.19437) (end 180.30237 131.92) (width 0.2) (layer "F.Cu") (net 2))
 (segment (start 174.505372 133.501) (end 173.919 132.914628) (width 0.2) (layer "F.Cu") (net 2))
 (segment (start 173.919 132.914628) (end 173.919 126.22337) (width 0.2) (layer "F.Cu") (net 2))
 (segment (start 181.876 121.496) (end 178.26 117.88) (width 0.2) (layer "F.Cu") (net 11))
 (segment (start 197 132.5) (end 197 122.739274) (width 0.2) (layer "F.Cu") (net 11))
 (segment (start 195.756726 121.496) (end 181.876 121.496) (width 0.2) (layer "F.Cu") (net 11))
 (segment (start 197 122.739274) (end 195.756726 121.496) (width 0.2) (layer "F.Cu") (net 11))
 (segment (start 191.92 132.5) (end 191.92 136.42) (width 0.2) (layer "F.Cu") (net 3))
 (segment (start 191.92 136.42) (end 197 141.5) (width 0.2) (layer "F.Cu") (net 3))
 (segment (start 178.26 110.26) (end 179.323 111.323) (width 0.2) (layer "F.Cu") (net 8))
 (segment (start 178.70031 113.863) (end 170.9701 113.863) (width 0.2) (layer "F.Cu") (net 8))
 (segment (start 179.323 111.323) (end 179.323 113.24031) (width 0.2) (layer "F.Cu") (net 8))
 (segment (start 164.6261 107.519) (end 163.051 107.519) (width 0.2) (layer "F.Cu") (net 8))
 (segment (start 163.051 107.519) (end 157.11 113.46) (width 0.2) (layer "F.Cu") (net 8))
 (segment (start 170.9701 113.863) (end 164.6261 107.519) (width 0.2) (layer "F.Cu") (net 8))
 (segment (start 179.323 113.24031) (end 178.70031 113.863) (width 0.2) (layer "F.Cu") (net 8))
 (segment (start 197.500578 142.7085) (end 198.402 141.807078) (width 0.2) (layer "F.Cu") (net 4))
 (segment (start 156.59747 134.059) (end 156.33747 133.799) (width 0.2) (layer "F.Cu") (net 4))
 (segment (start 183.3975 152.5625) (end 194.46 141.5) (width 0.2) (layer "F.Cu") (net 4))
 (segment (start 195.6685 142.7085) (end 197.500578 142.7085) (width 0.2) (layer "F.Cu") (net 4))
 (segment (start 163.46 110.92) (end 162.675184 110.92) (width 0.2) (layer "F.Cu") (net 4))
 (segment (start 194.46 141.5) (end 195.6685 142.7085) (width 0.2) (layer "F.Cu") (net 4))
 (segment (start 163.46 110.92) (end 163.46 129.92) (width 0.2) (layer "F.Cu") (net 4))
 (segment (start 164.095184 141.5) (end 173.81 141.5) (width 0.2) (layer "F.Cu") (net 4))
 (segment (start 163.46 148.92) (end 157.671 143.131) (width 0.2) (layer "F.Cu") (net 4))
 (segment (start 166.39 148.92) (end 163.46 148.92) (width 0.2) (layer "F.Cu") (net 4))
 (segment (start 173.81 141.5) (end 166.39 148.92) (width 0.2) (layer "F.Cu") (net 4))
 (segment (start 154.639 143.0176) (end 164.1839 152.5625) (width 0.2) (layer "F.Cu") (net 4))
 (segment (start 157.671 143.131) (end 157.671 134.2939) (width 0.2) (layer "F.Cu") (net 4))
 (segment (start 184.7675 142.3075) (end 185.1254 142.3075) (width 0.2) (layer "F.Cu") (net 4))
 (segment (start 157.4361 134.059) (end 158.569 135.1919) (width 0.2) (layer "F.Cu") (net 4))
 (segment (start 164.1839 152.5625) (end 183.3975 152.5625) (width 0.2) (layer "F.Cu") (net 4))
 (segment (start 158.569 135.1919) (end 158.569 135.973816) (width 0.2) (layer "F.Cu") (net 4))
 (segment (start 163.46 129.92) (end 161.904366 129.92) (width 0.2) (layer "F.Cu") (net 4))
 (segment (start 164.1839 152.5625) (end 175.047 152.5625) (width 0.2) (layer "F.Cu") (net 4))
 (segment (start 154.639 134.50253) (end 154.639 143.0176) (width 0.2) (layer "F.Cu") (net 4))
 (segment (start 198.402 116.867) (end 194.335 112.8) (width 0.2) (layer "F.Cu") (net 4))
 (segment (start 155.34253 133.799) (end 154.639 134.50253) (width 0.2) (layer "F.Cu") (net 4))
 (segment (start 175.047 152.5625) (end 184.5 143.1095) (width 0.2) (layer "F.Cu") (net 4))
 (segment (start 155.34253 133.799) (end 154.820765 134.320765) (width 0.2) (layer "F.Cu") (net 4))
 (segment (start 198.402 141.807078) (end 198.402 116.867) (width 0.2) (layer "F.Cu") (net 4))
 (segment (start 158.569 135.973816) (end 164.095184 141.5) (width 0.2) (layer "F.Cu") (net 4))
 (segment (start 156.33747 133.799) (end 155.34253 133.799) (width 0.2) (layer "F.Cu") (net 4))
 (segment (start 183.96 141.5) (end 184.7675 142.3075) (width 0.2) (layer "F.Cu") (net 4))
 (segment (start 161.904366 129.92) (end 157.765366 134.059) (width 0.2) (layer "F.Cu") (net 4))
 (segment (start 157.671 134.2939) (end 157.4361 134.059) (width 0.2) (layer "F.Cu") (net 4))
 (segment (start 157.4361 134.059) (end 156.59747 134.059) (width 0.2) (layer "F.Cu") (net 4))
 (segment (start 157.765366 134.059) (end 156.59747 134.059) (width 0.2) (layer "F.Cu") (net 4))
 (segment (start 155.709 112.879686) (end 161.470686 107.118) (width 0.2) (layer "F.Cu") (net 9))
 (segment (start 155.709 114.040314) (end 155.709 112.879686) (width 0.2) (layer "F.Cu") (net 9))
 (segment (start 157.11 115.441314) (end 155.709 114.040314) (width 0.2) (layer "F.Cu") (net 9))
 (segment (start 171.964374 107.118) (end 177.646374 112.8) (width 0.2) (layer "F.Cu") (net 9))
 (segment (start 157.11 132.46) (end 157.11 115.441314) (width 0.2) (layer "F.Cu") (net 9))
 (segment (start 177.646374 112.8) (end 178.26 112.8) (width 0.2) (layer "F.Cu") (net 9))
 (segment (start 161.470686 107.118) (end 171.964374 107.118) (width 0.2) (layer "F.Cu") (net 9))
 (segment (start 157.15 151.5) (end 157.5 151.5) (width 0.2) (layer "F.Cu") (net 7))
 (segment (start 157.11 151.46) (end 157.15 151.5) (width 0.2) (layer "F.Cu") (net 7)))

